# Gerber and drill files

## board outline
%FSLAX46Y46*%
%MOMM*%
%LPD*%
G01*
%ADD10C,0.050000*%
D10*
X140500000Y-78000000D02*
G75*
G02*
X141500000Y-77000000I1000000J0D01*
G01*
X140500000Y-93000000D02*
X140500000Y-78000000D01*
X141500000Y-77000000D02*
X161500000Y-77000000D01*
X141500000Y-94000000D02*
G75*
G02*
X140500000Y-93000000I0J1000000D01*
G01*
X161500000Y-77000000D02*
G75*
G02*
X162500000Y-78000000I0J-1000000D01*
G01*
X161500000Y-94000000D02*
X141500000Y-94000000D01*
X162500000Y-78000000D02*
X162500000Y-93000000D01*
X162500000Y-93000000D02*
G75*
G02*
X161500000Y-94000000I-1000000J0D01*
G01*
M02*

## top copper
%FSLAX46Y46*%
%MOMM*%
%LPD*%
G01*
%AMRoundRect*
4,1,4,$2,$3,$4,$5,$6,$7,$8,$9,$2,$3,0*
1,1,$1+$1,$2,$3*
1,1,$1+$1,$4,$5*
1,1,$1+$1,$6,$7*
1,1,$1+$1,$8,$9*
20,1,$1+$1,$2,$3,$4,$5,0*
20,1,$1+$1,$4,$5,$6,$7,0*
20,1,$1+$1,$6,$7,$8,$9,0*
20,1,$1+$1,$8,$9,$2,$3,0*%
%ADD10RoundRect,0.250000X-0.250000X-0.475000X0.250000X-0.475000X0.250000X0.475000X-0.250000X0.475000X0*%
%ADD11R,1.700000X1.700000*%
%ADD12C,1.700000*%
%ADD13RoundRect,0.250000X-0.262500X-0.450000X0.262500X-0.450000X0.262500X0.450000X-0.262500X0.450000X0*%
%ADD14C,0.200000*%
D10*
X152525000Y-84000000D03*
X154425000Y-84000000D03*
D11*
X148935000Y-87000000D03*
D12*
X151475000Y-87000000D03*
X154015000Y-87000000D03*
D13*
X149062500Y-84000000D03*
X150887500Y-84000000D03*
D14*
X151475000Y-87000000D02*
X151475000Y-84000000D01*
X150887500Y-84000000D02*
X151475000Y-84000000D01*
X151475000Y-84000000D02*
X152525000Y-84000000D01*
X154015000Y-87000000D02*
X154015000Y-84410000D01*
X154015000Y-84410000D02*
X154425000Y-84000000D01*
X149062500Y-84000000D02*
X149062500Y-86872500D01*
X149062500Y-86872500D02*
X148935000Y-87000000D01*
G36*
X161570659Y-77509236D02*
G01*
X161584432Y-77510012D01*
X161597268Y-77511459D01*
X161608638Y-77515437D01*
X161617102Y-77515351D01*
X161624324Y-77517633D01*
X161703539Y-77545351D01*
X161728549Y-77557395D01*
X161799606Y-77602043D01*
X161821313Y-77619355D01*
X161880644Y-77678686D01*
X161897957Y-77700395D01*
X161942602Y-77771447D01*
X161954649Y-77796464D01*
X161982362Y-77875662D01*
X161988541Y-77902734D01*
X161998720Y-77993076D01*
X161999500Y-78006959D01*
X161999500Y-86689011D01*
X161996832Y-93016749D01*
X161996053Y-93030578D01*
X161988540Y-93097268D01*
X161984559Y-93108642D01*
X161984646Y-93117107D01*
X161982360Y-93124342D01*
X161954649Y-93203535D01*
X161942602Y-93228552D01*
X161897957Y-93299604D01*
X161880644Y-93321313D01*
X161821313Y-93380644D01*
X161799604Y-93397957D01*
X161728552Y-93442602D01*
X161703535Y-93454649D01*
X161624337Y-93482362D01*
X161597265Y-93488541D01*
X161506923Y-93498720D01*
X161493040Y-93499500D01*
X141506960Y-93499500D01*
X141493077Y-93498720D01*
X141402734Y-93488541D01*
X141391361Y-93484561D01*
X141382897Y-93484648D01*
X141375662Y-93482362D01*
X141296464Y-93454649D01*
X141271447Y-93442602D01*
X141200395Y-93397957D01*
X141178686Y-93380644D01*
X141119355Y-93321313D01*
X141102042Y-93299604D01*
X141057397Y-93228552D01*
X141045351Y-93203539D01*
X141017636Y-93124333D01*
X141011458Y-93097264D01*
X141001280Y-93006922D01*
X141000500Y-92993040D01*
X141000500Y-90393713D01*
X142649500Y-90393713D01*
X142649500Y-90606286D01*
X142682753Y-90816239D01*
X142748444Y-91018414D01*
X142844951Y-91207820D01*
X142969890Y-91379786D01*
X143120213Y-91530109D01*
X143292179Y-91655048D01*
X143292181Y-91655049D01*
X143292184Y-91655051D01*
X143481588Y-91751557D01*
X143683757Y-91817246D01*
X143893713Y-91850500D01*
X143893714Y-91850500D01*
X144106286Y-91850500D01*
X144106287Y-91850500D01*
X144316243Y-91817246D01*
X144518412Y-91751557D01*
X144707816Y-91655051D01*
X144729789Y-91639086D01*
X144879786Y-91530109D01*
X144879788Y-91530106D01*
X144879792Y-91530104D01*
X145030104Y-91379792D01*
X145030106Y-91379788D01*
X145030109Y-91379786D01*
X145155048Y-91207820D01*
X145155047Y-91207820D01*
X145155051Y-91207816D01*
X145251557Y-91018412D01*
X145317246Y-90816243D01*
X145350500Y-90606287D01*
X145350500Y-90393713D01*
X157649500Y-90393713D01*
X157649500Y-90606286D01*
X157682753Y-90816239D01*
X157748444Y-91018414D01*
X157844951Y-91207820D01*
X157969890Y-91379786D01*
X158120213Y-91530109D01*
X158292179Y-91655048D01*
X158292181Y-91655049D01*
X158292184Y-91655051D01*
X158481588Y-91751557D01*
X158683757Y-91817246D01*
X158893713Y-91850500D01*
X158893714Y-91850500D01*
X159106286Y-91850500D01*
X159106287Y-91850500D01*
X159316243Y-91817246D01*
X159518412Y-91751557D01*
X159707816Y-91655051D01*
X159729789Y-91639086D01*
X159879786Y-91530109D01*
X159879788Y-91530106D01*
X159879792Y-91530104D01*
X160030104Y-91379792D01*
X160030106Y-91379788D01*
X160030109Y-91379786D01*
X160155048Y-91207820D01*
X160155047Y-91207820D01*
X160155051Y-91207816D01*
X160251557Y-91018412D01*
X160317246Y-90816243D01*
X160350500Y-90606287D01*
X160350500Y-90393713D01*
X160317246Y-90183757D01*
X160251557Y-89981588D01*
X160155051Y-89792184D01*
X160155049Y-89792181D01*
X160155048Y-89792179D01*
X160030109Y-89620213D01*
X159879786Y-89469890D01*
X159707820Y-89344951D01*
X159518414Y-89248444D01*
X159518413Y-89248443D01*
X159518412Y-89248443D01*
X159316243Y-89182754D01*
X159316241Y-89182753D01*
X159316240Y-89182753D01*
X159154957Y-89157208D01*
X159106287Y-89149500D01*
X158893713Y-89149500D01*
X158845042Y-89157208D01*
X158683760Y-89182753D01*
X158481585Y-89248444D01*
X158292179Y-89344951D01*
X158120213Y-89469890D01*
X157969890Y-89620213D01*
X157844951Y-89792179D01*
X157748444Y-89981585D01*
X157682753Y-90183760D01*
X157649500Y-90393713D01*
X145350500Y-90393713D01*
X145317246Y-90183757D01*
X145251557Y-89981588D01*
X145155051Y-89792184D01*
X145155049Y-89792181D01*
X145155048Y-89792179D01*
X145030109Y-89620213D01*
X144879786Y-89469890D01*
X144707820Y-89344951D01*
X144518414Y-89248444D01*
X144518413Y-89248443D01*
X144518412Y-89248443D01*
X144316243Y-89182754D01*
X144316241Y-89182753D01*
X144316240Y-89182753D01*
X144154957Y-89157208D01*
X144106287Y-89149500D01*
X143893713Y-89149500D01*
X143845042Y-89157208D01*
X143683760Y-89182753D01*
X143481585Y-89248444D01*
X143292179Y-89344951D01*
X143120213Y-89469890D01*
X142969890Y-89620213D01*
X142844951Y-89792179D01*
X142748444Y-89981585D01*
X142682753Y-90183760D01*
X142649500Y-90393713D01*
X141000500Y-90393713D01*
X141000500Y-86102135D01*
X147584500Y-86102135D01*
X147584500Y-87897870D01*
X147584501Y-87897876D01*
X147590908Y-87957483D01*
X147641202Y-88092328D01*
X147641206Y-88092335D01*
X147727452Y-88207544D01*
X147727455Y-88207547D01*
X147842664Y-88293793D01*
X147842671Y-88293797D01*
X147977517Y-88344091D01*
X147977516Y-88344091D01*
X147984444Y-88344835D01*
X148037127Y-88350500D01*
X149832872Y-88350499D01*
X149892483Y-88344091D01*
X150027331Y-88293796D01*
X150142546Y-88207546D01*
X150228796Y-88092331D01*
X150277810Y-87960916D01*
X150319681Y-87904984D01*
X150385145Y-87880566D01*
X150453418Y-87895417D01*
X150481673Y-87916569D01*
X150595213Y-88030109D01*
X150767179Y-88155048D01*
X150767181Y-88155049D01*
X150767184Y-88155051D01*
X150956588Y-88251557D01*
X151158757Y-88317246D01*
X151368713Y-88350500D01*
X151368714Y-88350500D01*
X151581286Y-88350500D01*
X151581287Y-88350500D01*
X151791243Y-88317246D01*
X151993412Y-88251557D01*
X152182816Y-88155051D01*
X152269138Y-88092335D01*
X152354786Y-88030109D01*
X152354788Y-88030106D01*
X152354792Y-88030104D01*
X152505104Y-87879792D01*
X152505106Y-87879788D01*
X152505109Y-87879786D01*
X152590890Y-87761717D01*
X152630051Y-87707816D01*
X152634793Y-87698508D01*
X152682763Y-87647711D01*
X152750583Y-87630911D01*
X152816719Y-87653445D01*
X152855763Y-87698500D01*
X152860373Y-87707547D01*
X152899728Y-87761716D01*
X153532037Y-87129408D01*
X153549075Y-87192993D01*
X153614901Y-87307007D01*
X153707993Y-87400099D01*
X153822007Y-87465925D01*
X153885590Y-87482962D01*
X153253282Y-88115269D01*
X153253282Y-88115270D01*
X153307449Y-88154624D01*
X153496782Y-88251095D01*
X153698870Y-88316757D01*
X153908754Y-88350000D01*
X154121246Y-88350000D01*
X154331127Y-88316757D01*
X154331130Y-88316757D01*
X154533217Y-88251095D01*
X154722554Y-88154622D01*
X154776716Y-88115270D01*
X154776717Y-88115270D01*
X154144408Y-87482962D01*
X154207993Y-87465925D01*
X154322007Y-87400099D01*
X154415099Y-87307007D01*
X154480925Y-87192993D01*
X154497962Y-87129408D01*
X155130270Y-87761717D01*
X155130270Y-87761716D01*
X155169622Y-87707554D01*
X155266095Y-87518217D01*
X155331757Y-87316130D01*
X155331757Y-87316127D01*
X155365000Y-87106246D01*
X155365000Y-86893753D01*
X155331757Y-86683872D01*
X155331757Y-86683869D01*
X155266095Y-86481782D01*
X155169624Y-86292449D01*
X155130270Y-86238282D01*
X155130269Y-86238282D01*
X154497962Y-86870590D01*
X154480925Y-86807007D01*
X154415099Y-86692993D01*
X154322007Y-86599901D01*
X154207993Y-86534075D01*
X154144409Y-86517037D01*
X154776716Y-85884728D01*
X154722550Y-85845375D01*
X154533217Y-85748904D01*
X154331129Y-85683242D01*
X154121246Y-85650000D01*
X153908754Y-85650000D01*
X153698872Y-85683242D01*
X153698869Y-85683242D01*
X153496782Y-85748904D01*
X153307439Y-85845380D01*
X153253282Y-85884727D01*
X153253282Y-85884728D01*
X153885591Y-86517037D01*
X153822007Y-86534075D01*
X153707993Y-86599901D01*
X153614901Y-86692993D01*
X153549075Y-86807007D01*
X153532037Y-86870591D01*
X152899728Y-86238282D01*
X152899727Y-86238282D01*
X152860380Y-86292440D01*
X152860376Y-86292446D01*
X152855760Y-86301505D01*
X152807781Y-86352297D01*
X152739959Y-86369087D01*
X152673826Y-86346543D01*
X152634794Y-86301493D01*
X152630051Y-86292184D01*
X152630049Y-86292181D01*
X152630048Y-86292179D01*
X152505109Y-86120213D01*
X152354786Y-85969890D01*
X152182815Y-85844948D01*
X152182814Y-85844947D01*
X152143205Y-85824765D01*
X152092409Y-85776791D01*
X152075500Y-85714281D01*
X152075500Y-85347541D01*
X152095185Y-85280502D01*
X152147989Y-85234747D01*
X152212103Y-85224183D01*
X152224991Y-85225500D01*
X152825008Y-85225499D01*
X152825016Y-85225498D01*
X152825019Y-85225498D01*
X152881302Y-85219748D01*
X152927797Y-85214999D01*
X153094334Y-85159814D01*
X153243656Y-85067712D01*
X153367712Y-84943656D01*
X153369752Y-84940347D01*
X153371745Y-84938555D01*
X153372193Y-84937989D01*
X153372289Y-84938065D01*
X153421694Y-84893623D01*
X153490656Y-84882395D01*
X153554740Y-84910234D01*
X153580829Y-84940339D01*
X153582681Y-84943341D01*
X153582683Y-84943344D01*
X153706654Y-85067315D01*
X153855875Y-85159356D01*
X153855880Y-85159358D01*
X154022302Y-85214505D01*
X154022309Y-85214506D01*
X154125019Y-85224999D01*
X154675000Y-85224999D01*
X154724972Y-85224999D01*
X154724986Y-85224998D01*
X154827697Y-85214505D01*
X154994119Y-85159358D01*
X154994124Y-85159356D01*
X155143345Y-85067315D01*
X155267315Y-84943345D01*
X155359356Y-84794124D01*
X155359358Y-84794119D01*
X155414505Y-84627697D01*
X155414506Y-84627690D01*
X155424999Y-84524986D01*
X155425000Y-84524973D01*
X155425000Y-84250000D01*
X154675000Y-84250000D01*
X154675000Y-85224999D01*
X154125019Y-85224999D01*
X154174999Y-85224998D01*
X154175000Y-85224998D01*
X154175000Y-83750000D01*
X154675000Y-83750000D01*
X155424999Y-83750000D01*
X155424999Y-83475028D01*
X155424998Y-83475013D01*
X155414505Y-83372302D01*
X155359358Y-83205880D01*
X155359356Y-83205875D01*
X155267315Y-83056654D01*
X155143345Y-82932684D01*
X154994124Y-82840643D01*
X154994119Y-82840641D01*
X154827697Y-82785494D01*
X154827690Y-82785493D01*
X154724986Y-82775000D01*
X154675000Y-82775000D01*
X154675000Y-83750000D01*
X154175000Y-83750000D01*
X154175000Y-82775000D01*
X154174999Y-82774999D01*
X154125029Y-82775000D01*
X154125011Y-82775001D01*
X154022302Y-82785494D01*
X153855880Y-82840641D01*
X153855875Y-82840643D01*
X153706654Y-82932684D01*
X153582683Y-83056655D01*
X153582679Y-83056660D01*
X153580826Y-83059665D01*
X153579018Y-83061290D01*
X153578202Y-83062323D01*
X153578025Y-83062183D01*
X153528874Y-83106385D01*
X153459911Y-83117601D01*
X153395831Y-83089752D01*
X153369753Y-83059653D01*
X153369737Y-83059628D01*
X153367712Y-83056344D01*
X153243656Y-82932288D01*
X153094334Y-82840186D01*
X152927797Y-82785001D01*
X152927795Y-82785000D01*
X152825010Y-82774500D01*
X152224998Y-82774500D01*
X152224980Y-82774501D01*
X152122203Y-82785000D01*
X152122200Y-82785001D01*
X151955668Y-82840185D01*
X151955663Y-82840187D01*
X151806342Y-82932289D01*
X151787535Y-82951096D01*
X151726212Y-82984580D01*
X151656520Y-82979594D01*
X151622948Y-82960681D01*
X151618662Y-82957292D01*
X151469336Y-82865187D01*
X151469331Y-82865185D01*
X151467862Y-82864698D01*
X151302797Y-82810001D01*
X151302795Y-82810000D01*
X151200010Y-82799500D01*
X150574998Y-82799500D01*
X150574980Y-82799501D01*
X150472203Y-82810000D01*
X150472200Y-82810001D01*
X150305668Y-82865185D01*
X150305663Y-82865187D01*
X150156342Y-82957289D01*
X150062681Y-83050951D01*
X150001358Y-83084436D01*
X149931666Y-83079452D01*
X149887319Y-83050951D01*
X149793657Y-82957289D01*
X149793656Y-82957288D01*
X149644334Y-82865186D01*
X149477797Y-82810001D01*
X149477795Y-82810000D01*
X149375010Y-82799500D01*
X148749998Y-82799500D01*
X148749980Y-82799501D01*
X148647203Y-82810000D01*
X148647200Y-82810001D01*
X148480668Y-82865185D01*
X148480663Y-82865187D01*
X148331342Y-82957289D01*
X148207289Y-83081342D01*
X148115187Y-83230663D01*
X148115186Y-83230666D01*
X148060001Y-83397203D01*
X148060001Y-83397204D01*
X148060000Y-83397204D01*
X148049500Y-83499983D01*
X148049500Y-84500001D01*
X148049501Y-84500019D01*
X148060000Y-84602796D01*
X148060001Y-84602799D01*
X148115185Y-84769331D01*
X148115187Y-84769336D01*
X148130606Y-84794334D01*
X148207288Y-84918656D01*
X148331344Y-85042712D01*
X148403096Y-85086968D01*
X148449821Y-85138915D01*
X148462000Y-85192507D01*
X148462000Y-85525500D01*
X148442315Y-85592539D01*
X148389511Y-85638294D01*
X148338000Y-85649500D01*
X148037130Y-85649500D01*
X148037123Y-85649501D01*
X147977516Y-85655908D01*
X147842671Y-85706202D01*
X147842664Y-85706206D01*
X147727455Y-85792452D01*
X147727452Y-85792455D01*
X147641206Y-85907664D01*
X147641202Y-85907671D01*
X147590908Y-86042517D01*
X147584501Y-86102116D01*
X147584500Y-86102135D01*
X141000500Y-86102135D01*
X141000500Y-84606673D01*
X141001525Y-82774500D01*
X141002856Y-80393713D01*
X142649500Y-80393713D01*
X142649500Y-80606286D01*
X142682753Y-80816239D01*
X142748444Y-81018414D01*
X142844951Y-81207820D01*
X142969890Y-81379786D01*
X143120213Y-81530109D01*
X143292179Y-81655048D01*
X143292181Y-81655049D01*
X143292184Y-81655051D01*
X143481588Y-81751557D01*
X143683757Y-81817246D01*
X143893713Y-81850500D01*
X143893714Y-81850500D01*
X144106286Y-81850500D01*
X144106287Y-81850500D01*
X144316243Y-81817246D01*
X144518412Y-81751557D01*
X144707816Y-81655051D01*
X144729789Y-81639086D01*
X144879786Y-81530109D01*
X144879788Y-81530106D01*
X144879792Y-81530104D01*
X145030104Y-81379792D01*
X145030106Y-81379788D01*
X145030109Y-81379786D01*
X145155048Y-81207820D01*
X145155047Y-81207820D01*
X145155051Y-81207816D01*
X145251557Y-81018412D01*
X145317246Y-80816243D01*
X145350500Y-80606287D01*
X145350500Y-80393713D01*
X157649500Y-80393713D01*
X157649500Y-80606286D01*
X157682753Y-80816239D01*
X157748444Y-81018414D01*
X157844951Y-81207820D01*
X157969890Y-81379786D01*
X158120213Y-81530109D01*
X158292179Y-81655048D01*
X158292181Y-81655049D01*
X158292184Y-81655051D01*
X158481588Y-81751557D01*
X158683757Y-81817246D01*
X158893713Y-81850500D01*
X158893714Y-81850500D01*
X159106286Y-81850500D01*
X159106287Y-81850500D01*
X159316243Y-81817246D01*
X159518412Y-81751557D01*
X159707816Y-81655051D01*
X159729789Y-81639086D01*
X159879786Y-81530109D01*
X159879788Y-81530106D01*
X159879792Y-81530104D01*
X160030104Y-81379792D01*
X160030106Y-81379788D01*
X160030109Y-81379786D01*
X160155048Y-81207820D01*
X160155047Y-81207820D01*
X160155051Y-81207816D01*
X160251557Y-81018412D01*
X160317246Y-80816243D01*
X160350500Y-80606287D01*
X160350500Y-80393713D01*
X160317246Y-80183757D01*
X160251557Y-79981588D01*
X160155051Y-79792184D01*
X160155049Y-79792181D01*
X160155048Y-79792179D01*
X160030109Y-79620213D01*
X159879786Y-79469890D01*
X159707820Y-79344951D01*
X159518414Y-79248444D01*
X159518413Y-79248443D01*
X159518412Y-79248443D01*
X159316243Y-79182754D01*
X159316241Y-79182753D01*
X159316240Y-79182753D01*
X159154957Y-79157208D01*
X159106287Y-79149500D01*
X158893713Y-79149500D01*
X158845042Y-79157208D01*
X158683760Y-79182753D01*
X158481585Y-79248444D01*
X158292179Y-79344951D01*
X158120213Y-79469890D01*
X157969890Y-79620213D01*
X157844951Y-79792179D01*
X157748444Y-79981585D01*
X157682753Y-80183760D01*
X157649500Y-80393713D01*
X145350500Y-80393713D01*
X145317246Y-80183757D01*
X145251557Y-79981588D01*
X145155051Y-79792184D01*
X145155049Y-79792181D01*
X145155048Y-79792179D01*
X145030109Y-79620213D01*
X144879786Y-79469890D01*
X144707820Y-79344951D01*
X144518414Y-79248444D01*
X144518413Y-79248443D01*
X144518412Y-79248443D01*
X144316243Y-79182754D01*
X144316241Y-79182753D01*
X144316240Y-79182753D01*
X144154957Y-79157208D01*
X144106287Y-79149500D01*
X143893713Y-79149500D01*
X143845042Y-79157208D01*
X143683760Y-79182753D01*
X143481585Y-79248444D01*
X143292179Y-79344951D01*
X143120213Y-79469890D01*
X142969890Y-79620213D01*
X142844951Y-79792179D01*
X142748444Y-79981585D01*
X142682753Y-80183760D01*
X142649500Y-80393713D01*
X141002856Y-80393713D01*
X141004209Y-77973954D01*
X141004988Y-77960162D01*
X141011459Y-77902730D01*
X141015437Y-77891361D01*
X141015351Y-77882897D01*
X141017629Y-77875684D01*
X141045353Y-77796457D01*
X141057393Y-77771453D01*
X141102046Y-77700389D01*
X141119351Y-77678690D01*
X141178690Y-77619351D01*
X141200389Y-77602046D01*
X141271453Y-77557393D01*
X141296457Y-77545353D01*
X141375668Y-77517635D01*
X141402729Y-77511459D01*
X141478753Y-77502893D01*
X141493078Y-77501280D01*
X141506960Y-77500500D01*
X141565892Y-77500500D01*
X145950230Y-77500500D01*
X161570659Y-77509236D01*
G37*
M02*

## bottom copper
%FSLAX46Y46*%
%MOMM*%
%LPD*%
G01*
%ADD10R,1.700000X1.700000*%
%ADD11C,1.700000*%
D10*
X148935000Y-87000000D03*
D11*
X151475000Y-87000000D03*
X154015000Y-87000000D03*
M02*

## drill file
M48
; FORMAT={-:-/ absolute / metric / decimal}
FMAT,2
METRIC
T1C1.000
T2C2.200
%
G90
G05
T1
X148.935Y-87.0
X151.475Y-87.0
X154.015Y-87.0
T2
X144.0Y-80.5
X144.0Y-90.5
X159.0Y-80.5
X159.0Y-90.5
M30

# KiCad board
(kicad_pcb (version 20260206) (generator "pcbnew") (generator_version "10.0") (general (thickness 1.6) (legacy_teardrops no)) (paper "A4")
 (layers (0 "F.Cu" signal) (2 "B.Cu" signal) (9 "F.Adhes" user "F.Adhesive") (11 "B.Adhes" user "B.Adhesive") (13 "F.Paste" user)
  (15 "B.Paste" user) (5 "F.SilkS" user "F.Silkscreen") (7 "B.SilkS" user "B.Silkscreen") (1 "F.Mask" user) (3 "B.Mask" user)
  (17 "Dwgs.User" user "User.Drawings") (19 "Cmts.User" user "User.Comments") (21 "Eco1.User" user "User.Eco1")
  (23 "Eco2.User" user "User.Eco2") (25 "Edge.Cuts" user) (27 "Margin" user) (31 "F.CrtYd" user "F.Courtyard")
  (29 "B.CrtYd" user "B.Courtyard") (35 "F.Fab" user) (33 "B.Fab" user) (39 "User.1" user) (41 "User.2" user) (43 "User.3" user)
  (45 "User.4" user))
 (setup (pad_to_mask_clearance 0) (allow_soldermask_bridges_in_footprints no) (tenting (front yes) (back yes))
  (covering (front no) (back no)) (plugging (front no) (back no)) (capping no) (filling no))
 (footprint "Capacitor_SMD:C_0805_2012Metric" (layer "F.Cu") (at 153.475 84)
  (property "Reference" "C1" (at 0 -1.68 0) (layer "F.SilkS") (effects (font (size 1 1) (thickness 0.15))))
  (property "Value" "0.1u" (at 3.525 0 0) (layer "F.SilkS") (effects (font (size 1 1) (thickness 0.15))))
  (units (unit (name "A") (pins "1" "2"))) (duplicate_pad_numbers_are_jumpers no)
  (pad "1" smd roundrect (at -0.95 0) (size 1 1.45) (layers "F.Cu" "F.Mask" "F.Paste") (roundrect_rratio 0.25) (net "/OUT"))
  (pad "2" smd roundrect (at 0.95 0) (size 1 1.45) (layers "F.Cu" "F.Mask" "F.Paste") (roundrect_rratio 0.25) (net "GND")))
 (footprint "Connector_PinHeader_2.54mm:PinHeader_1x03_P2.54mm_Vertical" (layer "F.Cu") (at 148.935 87 90)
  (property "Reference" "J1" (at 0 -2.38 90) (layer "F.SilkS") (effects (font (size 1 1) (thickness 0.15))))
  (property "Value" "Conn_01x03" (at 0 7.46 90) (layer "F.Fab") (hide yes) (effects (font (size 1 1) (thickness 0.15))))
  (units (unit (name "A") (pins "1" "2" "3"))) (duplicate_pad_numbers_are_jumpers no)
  (pad "1" thru_hole rect (at 0 0 90) (size 1.7 1.7) (drill 1) (layers "*.Cu" "*.Mask") (remove_unused_layers no) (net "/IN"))
  (pad "2" thru_hole circle (at 0 2.54 90) (size 1.7 1.7) (drill 1) (layers "*.Cu" "*.Mask") (remove_unused_layers no) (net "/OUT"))
  (pad "3" thru_hole circle (at 0 5.08 90) (size 1.7 1.7) (drill 1) (layers "*.Cu" "*.Mask") (remove_unused_layers no) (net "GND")))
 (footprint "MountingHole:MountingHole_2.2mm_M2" (layer "F.Cu") (at 144 90.5)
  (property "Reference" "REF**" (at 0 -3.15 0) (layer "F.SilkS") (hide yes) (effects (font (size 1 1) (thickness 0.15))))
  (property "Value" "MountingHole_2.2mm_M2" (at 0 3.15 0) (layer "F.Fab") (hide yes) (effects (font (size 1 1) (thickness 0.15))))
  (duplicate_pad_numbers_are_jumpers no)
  (pad "" np_thru_hole circle (at 0 0) (size 2.2 2.2) (drill 2.2) (layers "*.Cu" "*.Mask")))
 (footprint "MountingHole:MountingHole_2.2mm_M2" (layer "F.Cu") (at 159 80.5)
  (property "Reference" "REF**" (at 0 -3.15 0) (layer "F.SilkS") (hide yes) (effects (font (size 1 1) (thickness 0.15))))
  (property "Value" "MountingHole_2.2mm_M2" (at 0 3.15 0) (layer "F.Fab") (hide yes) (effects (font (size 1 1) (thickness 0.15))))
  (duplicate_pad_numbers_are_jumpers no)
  (pad "" np_thru_hole circle (at 0 0) (size 2.2 2.2) (drill 2.2) (layers "*.Cu" "*.Mask")))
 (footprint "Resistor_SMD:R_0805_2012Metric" (layer "F.Cu") (at 149.975 84)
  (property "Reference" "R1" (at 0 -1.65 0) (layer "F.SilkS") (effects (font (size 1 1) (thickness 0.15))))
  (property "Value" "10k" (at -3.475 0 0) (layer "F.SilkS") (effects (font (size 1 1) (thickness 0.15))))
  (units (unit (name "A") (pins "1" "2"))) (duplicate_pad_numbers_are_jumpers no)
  (pad "1" smd roundrect (at -0.9125 0) (size 1.025 1.4) (layers "F.Cu" "F.Mask" "F.Paste") (roundrect_rratio 0.243902) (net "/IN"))
  (pad "2" smd roundrect (at 0.9125 0) (size 1.025 1.4) (layers "F.Cu" "F.Mask" "F.Paste") (roundrect_rratio 0.243902) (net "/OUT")))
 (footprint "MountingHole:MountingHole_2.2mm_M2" (layer "F.Cu") (at 144 80.5)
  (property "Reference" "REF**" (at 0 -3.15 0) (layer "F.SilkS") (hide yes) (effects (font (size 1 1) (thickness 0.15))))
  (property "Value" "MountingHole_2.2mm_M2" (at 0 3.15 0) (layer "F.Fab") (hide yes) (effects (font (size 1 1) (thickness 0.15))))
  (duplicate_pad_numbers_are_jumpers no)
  (pad "" np_thru_hole circle (at 0 0) (size 2.2 2.2) (drill 2.2) (layers "*.Cu" "*.Mask")))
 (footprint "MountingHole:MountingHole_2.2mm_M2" (layer "F.Cu") (at 159 90.5)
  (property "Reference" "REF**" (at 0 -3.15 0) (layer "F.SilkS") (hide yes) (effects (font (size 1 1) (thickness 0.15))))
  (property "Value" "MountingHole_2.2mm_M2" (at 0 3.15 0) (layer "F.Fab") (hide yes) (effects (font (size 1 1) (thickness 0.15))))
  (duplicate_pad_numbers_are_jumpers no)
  (pad "" np_thru_hole circle (at 0 0) (size 2.2 2.2) (drill 2.2) (layers "*.Cu" "*.Mask")))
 (gr_arc (start 140.5 78) (mid 140.792893 77.292893) (end 141.5 77) (stroke (width 0.05) (type default)) (layer "Edge.Cuts"))
 (gr_line (start 140.5 93) (end 140.5 78) (stroke (width 0.05) (type default)) (layer "Edge.Cuts"))
 (gr_line (start 141.5 77) (end 161.5 77) (stroke (width 0.05) (type default)) (layer "Edge.Cuts"))
 (gr_arc (start 141.5 94) (mid 140.792893 93.707107) (end 140.5 93) (stroke (width 0.05) (type default)) (layer "Edge.Cuts"))
 (gr_arc (start 161.5 77) (mid 162.207107 77.292893) (end 162.5 78) (stroke (width 0.05) (type default)) (layer "Edge.Cuts"))
 (gr_line (start 161.5 94) (end 141.5 94) (stroke (width 0.05) (type default)) (layer "Edge.Cuts"))
 (gr_line (start 162.5 78) (end 162.5 93) (stroke (width 0.05) (type default)) (layer "Edge.Cuts"))
 (gr_arc (start 162.5 93) (mid 162.207107 93.707107) (end 161.5 94) (stroke (width 0.05) (type default)) (layer "Edge.Cuts"))
 (segment (start 151.475 87) (end 151.475 84) (width 0.2) (layer "F.Cu") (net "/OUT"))
 (segment (start 150.8875 84) (end 151.475 84) (width 0.2) (layer "F.Cu") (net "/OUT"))
 (segment (start 151.475 84) (end 152.525 84) (width 0.2) (layer "F.Cu") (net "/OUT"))
 (segment (start 154.015 87) (end 154.015 84.41) (width 0.2) (layer "F.Cu") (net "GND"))
 (segment (start 154.015 84.41) (end 154.425 84) (width 0.2) (layer "F.Cu") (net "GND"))
 (segment (start 149.0625 84) (end 149.0625 86.8725) (width 0.2) (layer "F.Cu") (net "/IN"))
 (segment (start 149.0625 86.8725) (end 148.935 87) (width 0.2) (layer "F.Cu") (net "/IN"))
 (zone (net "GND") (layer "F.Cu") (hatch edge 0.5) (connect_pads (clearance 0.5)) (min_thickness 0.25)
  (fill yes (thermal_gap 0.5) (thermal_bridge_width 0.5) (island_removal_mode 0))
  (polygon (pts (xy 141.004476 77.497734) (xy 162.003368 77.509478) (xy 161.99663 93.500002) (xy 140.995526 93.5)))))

